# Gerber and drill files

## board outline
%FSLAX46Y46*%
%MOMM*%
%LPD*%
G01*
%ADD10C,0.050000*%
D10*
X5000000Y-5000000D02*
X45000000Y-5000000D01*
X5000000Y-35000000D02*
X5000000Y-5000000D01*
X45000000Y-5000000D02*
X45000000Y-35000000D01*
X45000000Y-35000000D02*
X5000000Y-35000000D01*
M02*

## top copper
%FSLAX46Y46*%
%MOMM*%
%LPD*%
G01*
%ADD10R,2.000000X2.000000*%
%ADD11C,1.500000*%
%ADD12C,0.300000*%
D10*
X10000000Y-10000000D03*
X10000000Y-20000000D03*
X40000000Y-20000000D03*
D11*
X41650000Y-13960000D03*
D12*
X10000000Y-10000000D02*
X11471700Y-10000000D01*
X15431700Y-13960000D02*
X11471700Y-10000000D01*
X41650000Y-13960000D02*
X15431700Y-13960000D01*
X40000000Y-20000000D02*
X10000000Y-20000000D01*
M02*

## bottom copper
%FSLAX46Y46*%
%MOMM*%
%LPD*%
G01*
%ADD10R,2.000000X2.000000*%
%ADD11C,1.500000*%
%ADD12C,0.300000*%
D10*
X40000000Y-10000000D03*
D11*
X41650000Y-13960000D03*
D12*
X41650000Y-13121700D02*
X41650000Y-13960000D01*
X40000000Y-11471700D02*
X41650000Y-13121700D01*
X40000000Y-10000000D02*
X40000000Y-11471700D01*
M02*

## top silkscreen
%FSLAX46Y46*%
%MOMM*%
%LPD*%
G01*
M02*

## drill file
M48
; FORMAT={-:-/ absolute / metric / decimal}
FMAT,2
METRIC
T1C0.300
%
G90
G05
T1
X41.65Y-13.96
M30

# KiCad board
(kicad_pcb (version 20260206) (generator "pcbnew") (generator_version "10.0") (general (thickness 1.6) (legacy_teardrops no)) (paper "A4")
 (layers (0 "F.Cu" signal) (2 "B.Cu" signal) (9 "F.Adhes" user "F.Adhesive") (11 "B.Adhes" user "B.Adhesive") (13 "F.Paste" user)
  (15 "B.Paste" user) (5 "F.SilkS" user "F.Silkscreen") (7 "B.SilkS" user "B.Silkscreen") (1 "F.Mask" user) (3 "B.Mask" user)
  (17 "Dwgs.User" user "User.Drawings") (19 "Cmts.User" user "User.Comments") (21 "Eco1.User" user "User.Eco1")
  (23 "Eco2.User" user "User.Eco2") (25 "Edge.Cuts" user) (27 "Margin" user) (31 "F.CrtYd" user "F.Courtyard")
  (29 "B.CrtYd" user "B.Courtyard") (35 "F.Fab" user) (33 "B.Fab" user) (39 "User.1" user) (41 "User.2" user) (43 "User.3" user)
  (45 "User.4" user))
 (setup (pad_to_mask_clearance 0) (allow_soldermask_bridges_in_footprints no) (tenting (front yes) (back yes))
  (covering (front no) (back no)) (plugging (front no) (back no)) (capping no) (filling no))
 (gr_line (start 5 5) (end 45 5) (stroke (width 0.05) (type default)) (layer "Edge.Cuts"))
 (gr_line (start 5 35) (end 5 5) (stroke (width 0.05) (type default)) (layer "Edge.Cuts"))
 (gr_line (start 45 5) (end 45 35) (stroke (width 0.05) (type default)) (layer "Edge.Cuts"))
 (gr_line (start 45 35) (end 5 35) (stroke (width 0.05) (type default)) (layer "Edge.Cuts"))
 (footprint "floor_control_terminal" (layer "F.Cu") (at 10 10)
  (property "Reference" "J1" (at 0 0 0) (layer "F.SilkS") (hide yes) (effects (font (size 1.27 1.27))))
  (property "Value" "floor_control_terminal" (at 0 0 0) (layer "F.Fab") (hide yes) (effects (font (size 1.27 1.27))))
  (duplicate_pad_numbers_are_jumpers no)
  (pad "1" smd rect (at 0 0) (size 2 2) (layers "F.Cu" "F.Paste" "F.Mask") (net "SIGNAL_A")))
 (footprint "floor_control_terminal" (layer "B.Cu") (at 40 10)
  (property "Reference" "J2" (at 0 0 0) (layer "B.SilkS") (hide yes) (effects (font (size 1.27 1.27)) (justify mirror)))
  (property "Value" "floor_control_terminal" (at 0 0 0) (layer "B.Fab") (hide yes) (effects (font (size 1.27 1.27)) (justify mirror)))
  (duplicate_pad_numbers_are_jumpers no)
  (pad "1" smd rect (at 0 0) (size 2 2) (layers "B.Cu" "B.Paste" "B.Mask") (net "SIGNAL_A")))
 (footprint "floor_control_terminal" (layer "F.Cu") (at 10 20)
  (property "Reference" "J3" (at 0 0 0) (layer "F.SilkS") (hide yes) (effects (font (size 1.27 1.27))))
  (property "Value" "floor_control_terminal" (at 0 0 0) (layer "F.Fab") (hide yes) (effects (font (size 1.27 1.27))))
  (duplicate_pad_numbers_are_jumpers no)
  (pad "1" smd rect (at 0 0) (size 2 2) (layers "F.Cu" "F.Paste" "F.Mask") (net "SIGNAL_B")))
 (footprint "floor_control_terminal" (layer "F.Cu") (at 40 20)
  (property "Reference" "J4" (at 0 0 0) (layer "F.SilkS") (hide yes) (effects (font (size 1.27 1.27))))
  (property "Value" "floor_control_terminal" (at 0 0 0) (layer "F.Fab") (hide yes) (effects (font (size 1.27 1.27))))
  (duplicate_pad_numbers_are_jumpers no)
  (pad "1" smd rect (at 0 0) (size 2 2) (layers "F.Cu" "F.Paste" "F.Mask") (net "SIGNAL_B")))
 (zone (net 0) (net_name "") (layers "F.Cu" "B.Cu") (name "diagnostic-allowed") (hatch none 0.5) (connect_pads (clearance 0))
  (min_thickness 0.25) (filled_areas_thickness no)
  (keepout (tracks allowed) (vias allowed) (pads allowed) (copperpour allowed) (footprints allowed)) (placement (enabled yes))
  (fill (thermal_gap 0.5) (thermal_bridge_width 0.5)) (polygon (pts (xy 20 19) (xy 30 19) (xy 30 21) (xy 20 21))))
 (segment (start 10 10) (end 11.4717 10) (width 0.3) (layer "F.Cu") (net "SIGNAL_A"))
 (segment (start 15.4317 13.96) (end 11.4717 10) (width 0.3) (layer "F.Cu") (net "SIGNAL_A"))
 (segment (start 41.65 13.96) (end 15.4317 13.96) (width 0.3) (layer "F.Cu") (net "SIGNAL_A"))
 (via (at 41.65 13.96) (size 1.5) (drill 0.3) (layers "F.Cu" "B.Cu") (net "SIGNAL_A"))
 (segment (start 41.65 13.1217) (end 41.65 13.96) (width 0.3) (layer "B.Cu") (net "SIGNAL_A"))
 (segment (start 40 11.4717) (end 41.65 13.1217) (width 0.3) (layer "B.Cu") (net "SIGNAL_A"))
 (segment (start 40 10) (end 40 11.4717) (width 0.3) (layer "B.Cu") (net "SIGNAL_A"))
 (segment (start 40 20) (end 10 20) (width 0.3) (layer "F.Cu") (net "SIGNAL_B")))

